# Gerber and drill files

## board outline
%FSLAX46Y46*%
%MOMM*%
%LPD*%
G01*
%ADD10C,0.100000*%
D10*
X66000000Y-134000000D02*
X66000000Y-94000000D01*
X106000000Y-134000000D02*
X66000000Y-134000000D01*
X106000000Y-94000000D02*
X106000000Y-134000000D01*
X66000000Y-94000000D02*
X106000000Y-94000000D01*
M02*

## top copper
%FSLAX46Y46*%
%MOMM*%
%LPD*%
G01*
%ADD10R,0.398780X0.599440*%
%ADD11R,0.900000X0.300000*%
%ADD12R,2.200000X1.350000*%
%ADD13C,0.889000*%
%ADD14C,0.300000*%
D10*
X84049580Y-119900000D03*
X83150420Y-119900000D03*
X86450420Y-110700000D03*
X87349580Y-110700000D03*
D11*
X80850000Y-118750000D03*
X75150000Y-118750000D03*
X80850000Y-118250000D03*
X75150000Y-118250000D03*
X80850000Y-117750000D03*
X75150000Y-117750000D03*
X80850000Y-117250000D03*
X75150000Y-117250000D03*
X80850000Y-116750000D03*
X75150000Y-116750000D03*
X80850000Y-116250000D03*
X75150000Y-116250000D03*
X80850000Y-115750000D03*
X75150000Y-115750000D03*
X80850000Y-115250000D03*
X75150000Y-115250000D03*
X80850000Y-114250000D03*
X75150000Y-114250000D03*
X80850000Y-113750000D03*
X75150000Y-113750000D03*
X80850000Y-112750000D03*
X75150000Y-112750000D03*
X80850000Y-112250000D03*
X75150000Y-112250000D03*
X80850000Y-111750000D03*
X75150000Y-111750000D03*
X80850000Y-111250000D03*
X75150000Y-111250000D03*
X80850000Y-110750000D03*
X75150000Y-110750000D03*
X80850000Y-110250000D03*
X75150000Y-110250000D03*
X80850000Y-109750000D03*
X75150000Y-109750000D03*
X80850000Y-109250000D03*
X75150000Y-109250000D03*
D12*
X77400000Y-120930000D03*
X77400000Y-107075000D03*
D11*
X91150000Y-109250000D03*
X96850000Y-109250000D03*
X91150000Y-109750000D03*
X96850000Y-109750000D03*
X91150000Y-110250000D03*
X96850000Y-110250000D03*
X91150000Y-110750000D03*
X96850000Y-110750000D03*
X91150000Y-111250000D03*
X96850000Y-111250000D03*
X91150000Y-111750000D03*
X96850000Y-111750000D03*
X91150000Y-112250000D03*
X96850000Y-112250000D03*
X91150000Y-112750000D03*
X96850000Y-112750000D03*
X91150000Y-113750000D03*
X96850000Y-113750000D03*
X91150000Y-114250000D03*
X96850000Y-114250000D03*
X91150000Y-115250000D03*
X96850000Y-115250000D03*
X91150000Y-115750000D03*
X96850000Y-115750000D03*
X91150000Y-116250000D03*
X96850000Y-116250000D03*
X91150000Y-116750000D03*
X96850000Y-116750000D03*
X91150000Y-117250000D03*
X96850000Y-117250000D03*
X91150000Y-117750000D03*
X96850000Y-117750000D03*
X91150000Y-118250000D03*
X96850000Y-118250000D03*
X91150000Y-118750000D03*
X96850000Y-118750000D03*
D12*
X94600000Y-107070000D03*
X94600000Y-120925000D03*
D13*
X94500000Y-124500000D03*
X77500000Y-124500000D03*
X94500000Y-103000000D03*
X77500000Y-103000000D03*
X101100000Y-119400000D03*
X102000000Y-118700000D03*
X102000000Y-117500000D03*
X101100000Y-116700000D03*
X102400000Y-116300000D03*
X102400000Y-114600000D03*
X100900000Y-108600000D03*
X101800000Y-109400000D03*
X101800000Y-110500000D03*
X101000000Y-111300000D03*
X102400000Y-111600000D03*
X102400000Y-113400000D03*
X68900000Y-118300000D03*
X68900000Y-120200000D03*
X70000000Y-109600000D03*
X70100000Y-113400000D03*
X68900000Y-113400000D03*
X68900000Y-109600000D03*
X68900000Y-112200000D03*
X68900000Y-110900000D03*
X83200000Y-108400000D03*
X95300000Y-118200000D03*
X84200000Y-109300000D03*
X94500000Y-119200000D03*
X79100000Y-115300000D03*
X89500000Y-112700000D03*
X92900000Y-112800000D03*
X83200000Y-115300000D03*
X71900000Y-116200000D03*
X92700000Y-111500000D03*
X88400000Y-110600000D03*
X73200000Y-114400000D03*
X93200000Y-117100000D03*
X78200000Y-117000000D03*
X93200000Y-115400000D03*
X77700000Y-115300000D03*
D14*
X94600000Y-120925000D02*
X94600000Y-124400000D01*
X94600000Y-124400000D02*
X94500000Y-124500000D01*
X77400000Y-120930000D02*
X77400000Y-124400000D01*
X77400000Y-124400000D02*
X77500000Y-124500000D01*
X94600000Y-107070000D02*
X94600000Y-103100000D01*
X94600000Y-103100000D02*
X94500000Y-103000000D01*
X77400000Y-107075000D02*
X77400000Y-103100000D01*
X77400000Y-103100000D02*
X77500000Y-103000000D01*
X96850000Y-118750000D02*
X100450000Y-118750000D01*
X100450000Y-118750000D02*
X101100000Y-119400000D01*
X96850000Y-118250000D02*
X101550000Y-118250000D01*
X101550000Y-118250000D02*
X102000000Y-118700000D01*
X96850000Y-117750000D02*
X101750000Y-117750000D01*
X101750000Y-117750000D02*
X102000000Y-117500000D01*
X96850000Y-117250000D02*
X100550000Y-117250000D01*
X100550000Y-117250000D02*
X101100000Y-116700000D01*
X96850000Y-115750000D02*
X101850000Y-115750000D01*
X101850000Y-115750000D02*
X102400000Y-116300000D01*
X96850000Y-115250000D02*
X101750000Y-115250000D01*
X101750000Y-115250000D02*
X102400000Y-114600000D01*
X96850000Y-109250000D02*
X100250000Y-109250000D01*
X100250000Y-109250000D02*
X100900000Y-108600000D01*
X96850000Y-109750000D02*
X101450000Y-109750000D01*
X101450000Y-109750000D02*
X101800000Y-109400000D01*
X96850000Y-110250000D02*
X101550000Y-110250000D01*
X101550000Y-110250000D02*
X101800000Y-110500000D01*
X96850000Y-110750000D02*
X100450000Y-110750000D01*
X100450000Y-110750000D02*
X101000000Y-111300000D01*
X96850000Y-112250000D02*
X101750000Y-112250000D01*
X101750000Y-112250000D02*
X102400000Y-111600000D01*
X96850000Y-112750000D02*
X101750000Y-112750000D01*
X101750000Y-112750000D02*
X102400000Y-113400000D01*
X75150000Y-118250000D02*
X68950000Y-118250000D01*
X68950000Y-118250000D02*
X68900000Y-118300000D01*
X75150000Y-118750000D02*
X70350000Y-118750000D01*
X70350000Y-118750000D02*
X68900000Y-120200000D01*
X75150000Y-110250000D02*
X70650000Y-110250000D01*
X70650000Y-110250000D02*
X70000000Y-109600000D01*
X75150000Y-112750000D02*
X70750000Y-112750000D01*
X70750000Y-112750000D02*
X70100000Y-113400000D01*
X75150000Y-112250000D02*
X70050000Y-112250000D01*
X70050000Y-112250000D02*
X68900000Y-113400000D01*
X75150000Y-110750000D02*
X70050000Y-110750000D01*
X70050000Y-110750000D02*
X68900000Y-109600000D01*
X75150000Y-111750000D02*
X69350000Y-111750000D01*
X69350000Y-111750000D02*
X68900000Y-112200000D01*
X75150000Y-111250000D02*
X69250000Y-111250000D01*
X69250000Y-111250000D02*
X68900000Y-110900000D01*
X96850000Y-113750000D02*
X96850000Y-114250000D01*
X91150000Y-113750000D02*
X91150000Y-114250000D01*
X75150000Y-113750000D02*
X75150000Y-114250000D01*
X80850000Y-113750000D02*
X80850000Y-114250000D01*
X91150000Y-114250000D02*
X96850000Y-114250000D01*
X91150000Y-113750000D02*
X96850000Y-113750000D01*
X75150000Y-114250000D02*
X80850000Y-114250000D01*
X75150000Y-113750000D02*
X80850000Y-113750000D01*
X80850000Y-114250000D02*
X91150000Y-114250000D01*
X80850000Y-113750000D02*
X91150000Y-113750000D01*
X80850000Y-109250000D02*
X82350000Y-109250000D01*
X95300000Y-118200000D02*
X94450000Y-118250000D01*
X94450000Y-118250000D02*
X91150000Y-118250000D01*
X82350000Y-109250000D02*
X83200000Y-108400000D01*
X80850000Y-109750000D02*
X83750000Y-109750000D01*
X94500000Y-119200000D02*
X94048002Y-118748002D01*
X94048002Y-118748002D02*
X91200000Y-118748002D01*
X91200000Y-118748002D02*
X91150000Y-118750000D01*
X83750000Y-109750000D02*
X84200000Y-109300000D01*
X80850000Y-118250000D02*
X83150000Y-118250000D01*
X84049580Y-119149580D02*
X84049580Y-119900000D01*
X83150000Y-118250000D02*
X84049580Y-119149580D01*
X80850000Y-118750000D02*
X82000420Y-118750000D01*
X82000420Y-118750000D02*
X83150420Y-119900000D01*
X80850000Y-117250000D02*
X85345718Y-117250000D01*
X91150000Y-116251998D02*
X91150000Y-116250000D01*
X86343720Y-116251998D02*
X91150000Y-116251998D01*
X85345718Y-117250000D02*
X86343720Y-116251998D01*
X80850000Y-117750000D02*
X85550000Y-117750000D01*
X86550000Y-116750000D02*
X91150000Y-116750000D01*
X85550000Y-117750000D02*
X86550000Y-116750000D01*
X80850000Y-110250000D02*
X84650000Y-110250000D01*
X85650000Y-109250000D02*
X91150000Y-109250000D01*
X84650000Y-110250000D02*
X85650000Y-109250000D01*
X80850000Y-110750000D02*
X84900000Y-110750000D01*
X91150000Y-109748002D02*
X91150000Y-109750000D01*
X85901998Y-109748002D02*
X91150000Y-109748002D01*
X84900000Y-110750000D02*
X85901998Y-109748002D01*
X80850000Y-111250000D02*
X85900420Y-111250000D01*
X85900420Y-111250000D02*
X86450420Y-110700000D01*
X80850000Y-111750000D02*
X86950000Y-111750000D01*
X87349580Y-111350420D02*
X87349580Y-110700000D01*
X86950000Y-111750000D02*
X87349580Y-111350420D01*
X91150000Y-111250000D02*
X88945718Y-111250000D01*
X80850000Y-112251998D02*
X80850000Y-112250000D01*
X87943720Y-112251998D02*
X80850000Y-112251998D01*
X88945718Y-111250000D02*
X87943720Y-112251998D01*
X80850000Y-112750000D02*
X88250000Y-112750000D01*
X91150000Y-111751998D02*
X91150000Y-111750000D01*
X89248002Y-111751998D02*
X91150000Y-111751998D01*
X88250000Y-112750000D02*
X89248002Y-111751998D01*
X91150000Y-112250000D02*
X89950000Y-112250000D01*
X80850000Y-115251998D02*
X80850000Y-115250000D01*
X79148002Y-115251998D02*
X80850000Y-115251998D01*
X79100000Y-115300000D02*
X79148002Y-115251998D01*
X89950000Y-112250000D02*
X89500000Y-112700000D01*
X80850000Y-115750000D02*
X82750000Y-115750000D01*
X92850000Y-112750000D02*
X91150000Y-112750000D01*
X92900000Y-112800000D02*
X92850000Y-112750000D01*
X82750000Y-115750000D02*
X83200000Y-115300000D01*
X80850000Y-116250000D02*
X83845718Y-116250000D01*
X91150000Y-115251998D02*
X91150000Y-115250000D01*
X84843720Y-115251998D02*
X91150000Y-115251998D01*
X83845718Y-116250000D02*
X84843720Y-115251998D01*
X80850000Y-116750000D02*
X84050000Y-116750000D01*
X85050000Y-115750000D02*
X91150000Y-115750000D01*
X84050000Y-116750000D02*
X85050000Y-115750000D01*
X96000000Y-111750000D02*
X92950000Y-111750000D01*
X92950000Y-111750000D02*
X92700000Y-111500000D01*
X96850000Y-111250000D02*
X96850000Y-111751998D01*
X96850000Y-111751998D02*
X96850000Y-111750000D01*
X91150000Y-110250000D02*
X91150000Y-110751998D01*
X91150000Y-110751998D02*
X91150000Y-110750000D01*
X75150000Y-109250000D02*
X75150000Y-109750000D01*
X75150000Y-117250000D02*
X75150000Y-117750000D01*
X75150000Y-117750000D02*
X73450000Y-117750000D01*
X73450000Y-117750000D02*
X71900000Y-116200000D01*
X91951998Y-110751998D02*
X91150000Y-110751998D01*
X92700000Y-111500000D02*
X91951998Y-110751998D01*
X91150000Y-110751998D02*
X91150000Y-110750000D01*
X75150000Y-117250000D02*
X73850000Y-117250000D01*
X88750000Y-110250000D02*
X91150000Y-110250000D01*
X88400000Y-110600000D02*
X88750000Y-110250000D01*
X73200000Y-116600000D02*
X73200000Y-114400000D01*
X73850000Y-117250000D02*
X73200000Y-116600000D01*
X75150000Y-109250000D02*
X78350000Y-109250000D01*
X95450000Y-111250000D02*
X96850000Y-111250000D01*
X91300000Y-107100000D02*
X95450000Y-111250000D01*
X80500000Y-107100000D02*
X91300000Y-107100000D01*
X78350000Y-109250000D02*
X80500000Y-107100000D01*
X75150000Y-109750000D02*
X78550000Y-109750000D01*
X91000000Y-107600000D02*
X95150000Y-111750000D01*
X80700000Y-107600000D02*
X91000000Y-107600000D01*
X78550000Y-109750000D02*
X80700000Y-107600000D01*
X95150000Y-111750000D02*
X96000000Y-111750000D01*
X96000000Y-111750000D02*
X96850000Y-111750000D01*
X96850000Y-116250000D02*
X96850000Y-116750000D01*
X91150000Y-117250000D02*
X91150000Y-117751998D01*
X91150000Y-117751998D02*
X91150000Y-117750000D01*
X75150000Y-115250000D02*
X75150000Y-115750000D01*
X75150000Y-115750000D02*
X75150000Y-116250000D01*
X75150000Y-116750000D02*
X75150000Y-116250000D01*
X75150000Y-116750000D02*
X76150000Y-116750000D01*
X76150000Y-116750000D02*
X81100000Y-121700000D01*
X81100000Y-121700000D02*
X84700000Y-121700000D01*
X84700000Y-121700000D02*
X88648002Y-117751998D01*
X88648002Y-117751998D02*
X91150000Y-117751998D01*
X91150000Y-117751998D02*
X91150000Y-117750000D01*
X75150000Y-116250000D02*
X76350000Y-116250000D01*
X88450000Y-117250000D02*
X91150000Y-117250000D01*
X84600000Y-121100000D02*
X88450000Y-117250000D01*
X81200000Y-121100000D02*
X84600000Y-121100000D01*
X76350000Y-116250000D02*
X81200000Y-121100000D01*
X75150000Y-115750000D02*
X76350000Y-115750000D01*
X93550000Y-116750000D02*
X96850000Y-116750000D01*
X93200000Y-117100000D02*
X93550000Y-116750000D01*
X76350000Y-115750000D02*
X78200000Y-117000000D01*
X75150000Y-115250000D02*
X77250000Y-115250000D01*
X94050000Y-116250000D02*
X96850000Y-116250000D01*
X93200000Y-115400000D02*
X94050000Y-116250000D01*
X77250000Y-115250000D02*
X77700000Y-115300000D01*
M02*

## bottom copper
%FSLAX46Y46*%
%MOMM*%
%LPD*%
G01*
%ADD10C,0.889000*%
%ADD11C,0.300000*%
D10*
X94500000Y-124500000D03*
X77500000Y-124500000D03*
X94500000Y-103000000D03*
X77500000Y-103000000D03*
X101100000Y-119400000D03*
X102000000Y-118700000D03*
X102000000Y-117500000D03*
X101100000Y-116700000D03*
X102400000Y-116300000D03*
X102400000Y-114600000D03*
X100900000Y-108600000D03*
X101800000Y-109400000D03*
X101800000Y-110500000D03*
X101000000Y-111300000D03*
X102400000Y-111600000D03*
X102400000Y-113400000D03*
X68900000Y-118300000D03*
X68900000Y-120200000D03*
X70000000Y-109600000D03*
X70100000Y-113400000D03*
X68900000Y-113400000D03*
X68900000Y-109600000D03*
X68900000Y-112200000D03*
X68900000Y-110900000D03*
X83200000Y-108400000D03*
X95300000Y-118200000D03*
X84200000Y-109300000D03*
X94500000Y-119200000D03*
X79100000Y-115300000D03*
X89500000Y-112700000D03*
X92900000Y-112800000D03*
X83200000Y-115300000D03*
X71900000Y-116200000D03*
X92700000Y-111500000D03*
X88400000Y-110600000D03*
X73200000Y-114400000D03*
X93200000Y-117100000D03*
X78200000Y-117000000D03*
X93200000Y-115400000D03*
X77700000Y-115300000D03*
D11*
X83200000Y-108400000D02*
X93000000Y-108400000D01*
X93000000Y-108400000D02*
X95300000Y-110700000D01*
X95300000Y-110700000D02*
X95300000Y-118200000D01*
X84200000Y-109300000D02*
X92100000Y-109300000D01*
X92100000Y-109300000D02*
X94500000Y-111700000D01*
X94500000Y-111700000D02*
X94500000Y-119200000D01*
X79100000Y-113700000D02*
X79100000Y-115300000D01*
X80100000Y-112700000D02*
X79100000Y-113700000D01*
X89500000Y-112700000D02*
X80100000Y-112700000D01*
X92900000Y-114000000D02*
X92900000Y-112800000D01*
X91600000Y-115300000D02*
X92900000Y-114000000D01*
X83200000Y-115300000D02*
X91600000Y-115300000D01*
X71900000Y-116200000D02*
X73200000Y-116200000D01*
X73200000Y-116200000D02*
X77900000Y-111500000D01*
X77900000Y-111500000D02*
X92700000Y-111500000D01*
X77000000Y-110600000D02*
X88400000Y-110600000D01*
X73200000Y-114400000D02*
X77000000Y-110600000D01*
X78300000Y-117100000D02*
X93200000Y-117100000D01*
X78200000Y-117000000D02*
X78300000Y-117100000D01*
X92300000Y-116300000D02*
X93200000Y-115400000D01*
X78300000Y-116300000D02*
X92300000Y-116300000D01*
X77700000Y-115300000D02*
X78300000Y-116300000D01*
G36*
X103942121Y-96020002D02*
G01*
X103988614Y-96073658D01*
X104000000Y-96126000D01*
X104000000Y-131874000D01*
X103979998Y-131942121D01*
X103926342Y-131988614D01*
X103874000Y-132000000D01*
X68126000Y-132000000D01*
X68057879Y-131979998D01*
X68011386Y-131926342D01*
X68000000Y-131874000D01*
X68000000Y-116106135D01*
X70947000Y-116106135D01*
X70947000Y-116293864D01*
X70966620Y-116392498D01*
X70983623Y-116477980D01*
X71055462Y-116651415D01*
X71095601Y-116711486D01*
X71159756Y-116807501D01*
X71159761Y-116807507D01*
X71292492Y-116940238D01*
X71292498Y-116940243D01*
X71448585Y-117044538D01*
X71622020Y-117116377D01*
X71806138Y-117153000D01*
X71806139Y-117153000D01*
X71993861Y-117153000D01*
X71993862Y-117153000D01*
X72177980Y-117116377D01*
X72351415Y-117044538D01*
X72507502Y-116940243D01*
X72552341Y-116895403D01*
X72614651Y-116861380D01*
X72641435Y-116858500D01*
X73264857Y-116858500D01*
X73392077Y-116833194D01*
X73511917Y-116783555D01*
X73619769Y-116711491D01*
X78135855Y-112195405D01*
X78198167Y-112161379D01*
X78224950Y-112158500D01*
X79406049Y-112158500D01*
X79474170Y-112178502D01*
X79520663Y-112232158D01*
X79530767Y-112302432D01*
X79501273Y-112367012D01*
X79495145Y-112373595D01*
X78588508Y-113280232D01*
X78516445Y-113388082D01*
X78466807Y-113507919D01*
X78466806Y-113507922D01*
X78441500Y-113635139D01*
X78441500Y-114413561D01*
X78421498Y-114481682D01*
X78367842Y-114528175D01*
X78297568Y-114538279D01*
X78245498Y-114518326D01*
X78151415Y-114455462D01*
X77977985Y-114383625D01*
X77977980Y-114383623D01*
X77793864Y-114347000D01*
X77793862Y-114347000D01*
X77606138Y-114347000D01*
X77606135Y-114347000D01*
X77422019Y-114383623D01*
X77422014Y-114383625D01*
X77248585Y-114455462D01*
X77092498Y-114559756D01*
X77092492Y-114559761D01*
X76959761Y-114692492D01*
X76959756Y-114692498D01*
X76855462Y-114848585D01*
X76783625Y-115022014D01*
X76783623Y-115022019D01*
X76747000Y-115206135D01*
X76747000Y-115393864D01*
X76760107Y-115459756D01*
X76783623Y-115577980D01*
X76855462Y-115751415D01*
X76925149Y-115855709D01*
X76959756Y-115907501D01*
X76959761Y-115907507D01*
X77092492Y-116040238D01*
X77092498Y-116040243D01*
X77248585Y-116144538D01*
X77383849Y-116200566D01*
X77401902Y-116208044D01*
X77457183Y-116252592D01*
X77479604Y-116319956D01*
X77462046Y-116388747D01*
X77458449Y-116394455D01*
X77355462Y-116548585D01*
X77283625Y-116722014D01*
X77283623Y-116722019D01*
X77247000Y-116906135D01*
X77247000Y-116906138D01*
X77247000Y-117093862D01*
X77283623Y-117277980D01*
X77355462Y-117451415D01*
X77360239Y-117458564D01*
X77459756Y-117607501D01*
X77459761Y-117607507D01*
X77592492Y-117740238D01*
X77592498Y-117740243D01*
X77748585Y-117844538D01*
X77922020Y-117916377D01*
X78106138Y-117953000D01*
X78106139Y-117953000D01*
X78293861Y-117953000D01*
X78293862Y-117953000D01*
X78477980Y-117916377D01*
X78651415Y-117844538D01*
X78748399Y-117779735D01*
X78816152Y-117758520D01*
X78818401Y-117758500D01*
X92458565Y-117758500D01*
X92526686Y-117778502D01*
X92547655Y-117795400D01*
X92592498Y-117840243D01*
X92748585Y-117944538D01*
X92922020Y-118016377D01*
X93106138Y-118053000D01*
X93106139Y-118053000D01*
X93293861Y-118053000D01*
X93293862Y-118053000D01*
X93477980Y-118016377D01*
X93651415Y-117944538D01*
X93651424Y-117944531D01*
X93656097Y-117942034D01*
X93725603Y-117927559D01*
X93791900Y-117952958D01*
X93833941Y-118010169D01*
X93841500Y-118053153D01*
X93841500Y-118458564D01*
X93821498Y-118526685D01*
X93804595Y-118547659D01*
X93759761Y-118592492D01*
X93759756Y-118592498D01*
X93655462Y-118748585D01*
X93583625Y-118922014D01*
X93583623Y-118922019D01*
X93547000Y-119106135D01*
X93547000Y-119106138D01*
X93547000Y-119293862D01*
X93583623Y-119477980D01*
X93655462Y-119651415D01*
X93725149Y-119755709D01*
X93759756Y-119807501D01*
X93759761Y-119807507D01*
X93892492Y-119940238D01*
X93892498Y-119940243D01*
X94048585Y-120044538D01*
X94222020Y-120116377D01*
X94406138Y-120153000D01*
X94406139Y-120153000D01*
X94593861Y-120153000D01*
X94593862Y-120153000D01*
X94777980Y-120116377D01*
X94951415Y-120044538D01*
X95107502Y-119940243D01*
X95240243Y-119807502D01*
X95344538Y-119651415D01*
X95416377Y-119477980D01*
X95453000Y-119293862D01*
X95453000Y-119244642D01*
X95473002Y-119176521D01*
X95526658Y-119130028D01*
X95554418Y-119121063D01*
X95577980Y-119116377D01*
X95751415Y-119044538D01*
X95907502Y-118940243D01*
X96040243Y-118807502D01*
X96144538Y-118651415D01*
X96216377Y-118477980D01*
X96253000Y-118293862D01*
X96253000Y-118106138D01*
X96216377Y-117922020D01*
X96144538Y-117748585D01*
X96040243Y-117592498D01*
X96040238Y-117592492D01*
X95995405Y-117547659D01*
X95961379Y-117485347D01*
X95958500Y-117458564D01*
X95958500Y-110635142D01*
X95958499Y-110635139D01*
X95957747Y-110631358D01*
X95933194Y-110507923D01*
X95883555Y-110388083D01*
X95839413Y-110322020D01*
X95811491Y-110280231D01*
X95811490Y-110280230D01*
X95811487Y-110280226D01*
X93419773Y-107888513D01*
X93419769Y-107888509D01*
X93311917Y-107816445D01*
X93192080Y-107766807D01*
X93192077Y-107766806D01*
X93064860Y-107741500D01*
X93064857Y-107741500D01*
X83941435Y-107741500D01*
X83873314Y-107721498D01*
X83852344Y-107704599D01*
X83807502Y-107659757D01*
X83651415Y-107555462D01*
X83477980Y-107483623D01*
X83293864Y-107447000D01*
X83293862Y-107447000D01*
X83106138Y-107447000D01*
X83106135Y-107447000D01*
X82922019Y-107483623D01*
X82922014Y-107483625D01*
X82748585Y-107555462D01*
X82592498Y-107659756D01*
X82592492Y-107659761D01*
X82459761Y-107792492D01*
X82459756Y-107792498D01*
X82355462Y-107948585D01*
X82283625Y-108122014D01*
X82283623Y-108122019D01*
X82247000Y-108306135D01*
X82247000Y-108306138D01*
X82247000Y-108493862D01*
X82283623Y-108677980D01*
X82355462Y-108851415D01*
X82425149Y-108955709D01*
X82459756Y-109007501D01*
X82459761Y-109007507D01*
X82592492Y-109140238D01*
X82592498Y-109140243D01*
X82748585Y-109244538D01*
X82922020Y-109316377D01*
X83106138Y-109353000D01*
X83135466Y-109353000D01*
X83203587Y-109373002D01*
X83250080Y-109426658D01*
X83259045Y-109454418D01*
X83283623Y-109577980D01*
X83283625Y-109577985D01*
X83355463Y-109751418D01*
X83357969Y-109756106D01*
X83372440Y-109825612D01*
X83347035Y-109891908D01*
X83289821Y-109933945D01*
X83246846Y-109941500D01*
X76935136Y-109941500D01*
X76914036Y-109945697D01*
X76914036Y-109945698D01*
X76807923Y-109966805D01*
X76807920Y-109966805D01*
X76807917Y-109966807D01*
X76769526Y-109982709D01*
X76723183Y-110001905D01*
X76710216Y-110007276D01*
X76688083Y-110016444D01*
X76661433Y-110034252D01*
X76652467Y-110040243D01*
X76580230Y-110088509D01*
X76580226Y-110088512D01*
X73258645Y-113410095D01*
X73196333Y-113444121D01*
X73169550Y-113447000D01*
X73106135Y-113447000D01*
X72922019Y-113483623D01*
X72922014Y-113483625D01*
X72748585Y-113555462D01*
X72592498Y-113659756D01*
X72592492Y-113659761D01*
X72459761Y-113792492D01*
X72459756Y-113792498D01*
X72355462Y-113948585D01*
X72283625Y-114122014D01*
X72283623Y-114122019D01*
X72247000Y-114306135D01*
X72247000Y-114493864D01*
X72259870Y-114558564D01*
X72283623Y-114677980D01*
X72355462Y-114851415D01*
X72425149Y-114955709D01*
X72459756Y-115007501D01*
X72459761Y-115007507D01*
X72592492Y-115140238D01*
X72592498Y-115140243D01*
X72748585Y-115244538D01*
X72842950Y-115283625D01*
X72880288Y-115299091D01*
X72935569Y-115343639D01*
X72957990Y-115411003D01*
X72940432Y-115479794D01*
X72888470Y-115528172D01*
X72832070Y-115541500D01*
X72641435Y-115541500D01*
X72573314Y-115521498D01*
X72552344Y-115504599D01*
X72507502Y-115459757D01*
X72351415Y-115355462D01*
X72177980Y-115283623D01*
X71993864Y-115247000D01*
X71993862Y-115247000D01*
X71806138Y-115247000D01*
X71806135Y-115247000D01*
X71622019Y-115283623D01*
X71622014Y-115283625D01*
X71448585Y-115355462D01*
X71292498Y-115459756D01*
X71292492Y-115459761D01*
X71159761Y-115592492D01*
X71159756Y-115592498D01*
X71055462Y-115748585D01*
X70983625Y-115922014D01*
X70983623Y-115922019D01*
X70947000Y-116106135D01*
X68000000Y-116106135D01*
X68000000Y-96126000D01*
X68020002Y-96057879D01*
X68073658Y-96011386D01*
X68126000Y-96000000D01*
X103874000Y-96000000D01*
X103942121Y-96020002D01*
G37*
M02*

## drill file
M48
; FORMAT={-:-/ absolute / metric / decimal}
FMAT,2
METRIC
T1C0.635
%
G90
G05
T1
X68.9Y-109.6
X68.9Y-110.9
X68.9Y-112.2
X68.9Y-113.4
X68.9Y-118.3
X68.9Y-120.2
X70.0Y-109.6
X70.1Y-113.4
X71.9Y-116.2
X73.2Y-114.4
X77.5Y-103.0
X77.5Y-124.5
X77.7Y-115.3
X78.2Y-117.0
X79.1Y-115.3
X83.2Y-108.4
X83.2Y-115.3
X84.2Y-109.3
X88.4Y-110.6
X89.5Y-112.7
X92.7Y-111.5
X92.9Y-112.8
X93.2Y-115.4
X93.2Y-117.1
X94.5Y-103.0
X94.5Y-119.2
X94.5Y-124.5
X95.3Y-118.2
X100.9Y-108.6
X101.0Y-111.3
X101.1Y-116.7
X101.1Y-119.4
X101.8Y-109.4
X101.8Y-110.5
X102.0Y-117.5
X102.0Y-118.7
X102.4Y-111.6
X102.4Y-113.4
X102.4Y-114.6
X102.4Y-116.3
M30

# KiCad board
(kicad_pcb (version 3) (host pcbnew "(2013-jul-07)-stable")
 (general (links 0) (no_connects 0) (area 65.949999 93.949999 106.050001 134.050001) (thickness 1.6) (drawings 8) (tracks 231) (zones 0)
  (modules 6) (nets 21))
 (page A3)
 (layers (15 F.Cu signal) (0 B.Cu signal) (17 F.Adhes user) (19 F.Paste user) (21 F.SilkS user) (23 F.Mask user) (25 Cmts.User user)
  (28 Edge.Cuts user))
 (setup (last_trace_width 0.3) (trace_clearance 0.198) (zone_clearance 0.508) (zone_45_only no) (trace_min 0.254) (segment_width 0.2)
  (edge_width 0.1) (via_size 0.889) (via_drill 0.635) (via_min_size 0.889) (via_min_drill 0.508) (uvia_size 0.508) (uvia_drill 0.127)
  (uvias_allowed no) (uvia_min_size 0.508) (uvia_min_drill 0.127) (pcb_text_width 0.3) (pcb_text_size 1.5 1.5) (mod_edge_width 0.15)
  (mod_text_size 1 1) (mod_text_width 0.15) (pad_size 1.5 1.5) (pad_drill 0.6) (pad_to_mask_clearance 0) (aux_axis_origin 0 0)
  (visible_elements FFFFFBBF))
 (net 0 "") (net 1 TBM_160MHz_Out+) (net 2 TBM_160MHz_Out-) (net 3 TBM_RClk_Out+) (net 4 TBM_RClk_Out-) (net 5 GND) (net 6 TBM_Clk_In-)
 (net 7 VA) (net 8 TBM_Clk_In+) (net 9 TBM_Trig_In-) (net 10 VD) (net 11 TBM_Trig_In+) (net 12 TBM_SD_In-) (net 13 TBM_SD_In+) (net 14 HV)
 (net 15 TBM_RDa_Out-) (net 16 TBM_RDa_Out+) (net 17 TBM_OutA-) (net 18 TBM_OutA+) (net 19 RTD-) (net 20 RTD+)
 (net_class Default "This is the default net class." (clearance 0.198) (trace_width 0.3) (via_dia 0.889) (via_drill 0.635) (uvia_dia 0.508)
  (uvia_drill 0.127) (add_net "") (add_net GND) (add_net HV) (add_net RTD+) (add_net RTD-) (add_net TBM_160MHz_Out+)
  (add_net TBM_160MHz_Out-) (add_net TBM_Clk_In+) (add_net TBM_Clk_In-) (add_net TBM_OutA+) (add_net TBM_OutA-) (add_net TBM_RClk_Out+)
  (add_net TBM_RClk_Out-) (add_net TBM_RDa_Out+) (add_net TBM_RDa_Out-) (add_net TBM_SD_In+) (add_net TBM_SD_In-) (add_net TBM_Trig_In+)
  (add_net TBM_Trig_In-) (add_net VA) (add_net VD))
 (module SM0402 (layer F.Cu) (at 83.6 119.9 180)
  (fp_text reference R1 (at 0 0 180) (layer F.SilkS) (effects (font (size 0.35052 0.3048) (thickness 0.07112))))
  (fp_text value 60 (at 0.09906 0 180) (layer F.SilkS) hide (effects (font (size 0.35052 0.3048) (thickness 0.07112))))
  (pad 1 smd rect (at -0.44958 0 180) (size 0.39878 0.59944) (layers F.Cu F.Paste F.Mask) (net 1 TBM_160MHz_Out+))
  (pad 2 smd rect (at 0.44958 0 180) (size 0.39878 0.59944) (layers F.Cu F.Paste F.Mask) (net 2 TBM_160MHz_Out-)))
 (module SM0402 (layer F.Cu) (at 86.9 110.7)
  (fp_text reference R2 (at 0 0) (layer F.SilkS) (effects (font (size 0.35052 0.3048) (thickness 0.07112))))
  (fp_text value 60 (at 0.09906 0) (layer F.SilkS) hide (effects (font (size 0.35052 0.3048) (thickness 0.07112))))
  (pad 1 smd rect (at -0.44958 0) (size 0.39878 0.59944) (layers F.Cu F.Paste F.Mask) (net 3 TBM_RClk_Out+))
  (pad 2 smd rect (at 0.44958 0) (size 0.39878 0.59944) (layers F.Cu F.Paste F.Mask) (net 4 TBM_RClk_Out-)))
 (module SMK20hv (layer F.Cu) (at 78 114 90)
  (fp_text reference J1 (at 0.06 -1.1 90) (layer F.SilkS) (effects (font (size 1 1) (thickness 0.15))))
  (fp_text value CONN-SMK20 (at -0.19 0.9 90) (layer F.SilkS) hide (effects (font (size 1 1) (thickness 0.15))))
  (pad 1 smd rect (at -4.75 2.85 90) (size 0.3 0.9) (layers F.Cu F.Paste F.Mask) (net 2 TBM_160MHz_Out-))
  (pad 2 smd rect (at -4.75 -2.85 90) (size 0.3 0.9) (layers F.Cu F.Paste F.Mask) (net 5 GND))
  (pad 3 smd rect (at -4.25 2.85 90) (size 0.3 0.9) (layers F.Cu F.Paste F.Mask) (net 1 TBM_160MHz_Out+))
  (pad 4 smd rect (at -4.25 -2.85 90) (size 0.3 0.9) (layers F.Cu F.Paste F.Mask) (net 5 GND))
  (pad 5 smd rect (at -3.75 2.85 90) (size 0.3 0.9) (layers F.Cu F.Paste F.Mask) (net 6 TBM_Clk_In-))
  (pad 6 smd rect (at -3.75 -2.85 90) (size 0.3 0.9) (layers F.Cu F.Paste F.Mask) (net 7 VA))
  (pad 7 smd rect (at -3.25 2.85 90) (size 0.3 0.9) (layers F.Cu F.Paste F.Mask) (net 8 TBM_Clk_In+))
  (pad 8 smd rect (at -3.25 -2.85 90) (size 0.3 0.9) (layers F.Cu F.Paste F.Mask) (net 7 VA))
  (pad 9 smd rect (at -2.75 2.85 90) (size 0.3 0.9) (layers F.Cu F.Paste F.Mask) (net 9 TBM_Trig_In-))
  (pad 10 smd rect (at -2.75 -2.85 90) (size 0.3 0.9) (layers F.Cu F.Paste F.Mask) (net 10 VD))
  (pad 11 smd rect (at -2.25 2.85 90) (size 0.3 0.9) (layers F.Cu F.Paste F.Mask) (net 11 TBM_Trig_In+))
  (pad 12 smd rect (at -2.25 -2.85 90) (size 0.3 0.9) (layers F.Cu F.Paste F.Mask) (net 10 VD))
  (pad 13 smd rect (at -1.75 2.85 90) (size 0.3 0.9) (layers F.Cu F.Paste F.Mask) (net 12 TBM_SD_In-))
  (pad 14 smd rect (at -1.75 -2.85 90) (size 0.3 0.9) (layers F.Cu F.Paste F.Mask) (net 10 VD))
  (pad 15 smd rect (at -1.25 2.85 90) (size 0.3 0.9) (layers F.Cu F.Paste F.Mask) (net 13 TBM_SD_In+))
  (pad 16 smd rect (at -1.25 -2.85 90) (size 0.3 0.9) (layers F.Cu F.Paste F.Mask) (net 10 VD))
  (pad 19 smd rect (at -0.25 2.85 90) (size 0.3 0.9) (layers F.Cu F.Paste F.Mask) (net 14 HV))
  (pad 20 smd rect (at -0.25 -2.85 90) (size 0.3 0.9) (layers F.Cu F.Paste F.Mask) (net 14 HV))
  (pad 21 smd rect (at 0.25 2.85 90) (size 0.3 0.9) (layers F.Cu F.Paste F.Mask) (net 14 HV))
  (pad 22 smd rect (at 0.25 -2.85 90) (size 0.3 0.9) (layers F.Cu F.Paste F.Mask) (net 14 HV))
  (pad 25 smd rect (at 1.25 2.85 90) (size 0.3 0.9) (layers F.Cu F.Paste F.Mask) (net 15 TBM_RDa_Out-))
  (pad 26 smd rect (at 1.25 -2.85 90) (size 0.3 0.9) (layers F.Cu F.Paste F.Mask) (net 5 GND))
  (pad 27 smd rect (at 1.75 2.85 90) (size 0.3 0.9) (layers F.Cu F.Paste F.Mask) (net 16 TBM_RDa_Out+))
  (pad 28 smd rect (at 1.75 -2.85 90) (size 0.3 0.9) (layers F.Cu F.Paste F.Mask) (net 5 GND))
  (pad 29 smd rect (at 2.25 2.85 90) (size 0.3 0.9) (layers F.Cu F.Paste F.Mask) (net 4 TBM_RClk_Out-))
  (pad 30 smd rect (at 2.25 -2.85 90) (size 0.3 0.9) (layers F.Cu F.Paste F.Mask) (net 5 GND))
  (pad 31 smd rect (at 2.75 2.85 90) (size 0.3 0.9) (layers F.Cu F.Paste F.Mask) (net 3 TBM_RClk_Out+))
  (pad 32 smd rect (at 2.75 -2.85 90) (size 0.3 0.9) (layers F.Cu F.Paste F.Mask) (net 5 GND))
  (pad 33 smd rect (at 3.25 2.85 90) (size 0.3 0.9) (layers F.Cu F.Paste F.Mask) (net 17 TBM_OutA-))
  (pad 34 smd rect (at 3.25 -2.85 90) (size 0.3 0.9) (layers F.Cu F.Paste F.Mask) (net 5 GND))
  (pad 35 smd rect (at 3.75 2.85 90) (size 0.3 0.9) (layers F.Cu F.Paste F.Mask) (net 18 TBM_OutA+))
  (pad 36 smd rect (at 3.75 -2.85 90) (size 0.3 0.9) (layers F.Cu F.Paste F.Mask) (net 5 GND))
  (pad 37 smd rect (at 4.25 2.85 90) (size 0.3 0.9) (layers F.Cu F.Paste F.Mask) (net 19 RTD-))
  (pad 38 smd rect (at 4.25 -2.85 90) (size 0.3 0.9) (layers F.Cu F.Paste F.Mask) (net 7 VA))
  (pad 39 smd rect (at 4.75 2.85 90) (size 0.3 0.9) (layers F.Cu F.Paste F.Mask) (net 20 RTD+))
  (pad 40 smd rect (at 4.75 -2.85 90) (size 0.3 0.9) (layers F.Cu F.Paste F.Mask) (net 7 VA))
  (pad 41 smd rect (at -6.93 -0.6 90) (size 1.35 2.2) (layers F.Cu F.Paste F.Mask) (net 5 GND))
  (pad 42 smd rect (at 6.925 -0.6 90) (size 1.35 2.2) (layers F.Cu F.Paste F.Mask) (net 5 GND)))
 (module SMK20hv (layer F.Cu) (at 94 114 270)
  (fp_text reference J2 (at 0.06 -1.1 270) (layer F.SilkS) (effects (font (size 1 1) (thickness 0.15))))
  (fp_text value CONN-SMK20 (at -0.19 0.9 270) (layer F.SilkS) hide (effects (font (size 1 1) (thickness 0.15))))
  (pad 1 smd rect (at -4.75 2.85 270) (size 0.3 0.9) (layers F.Cu F.Paste F.Mask) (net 18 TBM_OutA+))
  (pad 2 smd rect (at -4.75 -2.85 270) (size 0.3 0.9) (layers F.Cu F.Paste F.Mask) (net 5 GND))
  (pad 3 smd rect (at -4.25 2.85 270) (size 0.3 0.9) (layers F.Cu F.Paste F.Mask) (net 17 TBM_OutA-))
  (pad 4 smd rect (at -4.25 -2.85 270) (size 0.3 0.9) (layers F.Cu F.Paste F.Mask) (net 5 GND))
  (pad 5 smd rect (at -3.75 2.85 270) (size 0.3 0.9) (layers F.Cu F.Paste F.Mask) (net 7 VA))
  (pad 6 smd rect (at -3.75 -2.85 270) (size 0.3 0.9) (layers F.Cu F.Paste F.Mask) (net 5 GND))
  (pad 7 smd rect (at -3.25 2.85 270) (size 0.3 0.9) (layers F.Cu F.Paste F.Mask) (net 7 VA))
  (pad 8 smd rect (at -3.25 -2.85 270) (size 0.3 0.9) (layers F.Cu F.Paste F.Mask) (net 5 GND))
  (pad 9 smd rect (at -2.75 2.85 270) (size 0.3 0.9) (layers F.Cu F.Paste F.Mask) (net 16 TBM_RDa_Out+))
  (pad 10 smd rect (at -2.75 -2.85 270) (size 0.3 0.9) (layers F.Cu F.Paste F.Mask) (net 7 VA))
  (pad 11 smd rect (at -2.25 2.85 270) (size 0.3 0.9) (layers F.Cu F.Paste F.Mask) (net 15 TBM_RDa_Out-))
  (pad 12 smd rect (at -2.25 -2.85 270) (size 0.3 0.9) (layers F.Cu F.Paste F.Mask) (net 7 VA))
  (pad 13 smd rect (at -1.75 2.85 270) (size 0.3 0.9) (layers F.Cu F.Paste F.Mask) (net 13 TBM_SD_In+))
  (pad 14 smd rect (at -1.75 -2.85 270) (size 0.3 0.9) (layers F.Cu F.Paste F.Mask) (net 5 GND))
  (pad 15 smd rect (at -1.25 2.85 270) (size 0.3 0.9) (layers F.Cu F.Paste F.Mask) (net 12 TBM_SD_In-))
  (pad 16 smd rect (at -1.25 -2.85 270) (size 0.3 0.9) (layers F.Cu F.Paste F.Mask) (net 5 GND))
  (pad 19 smd rect (at -0.25 2.85 270) (size 0.3 0.9) (layers F.Cu F.Paste F.Mask) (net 14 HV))
  (pad 20 smd rect (at -0.25 -2.85 270) (size 0.3 0.9) (layers F.Cu F.Paste F.Mask) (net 14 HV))
  (pad 21 smd rect (at 0.25 2.85 270) (size 0.3 0.9) (layers F.Cu F.Paste F.Mask) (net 14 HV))
  (pad 22 smd rect (at 0.25 -2.85 270) (size 0.3 0.9) (layers F.Cu F.Paste F.Mask) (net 14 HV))
  (pad 25 smd rect (at 1.25 2.85 270) (size 0.3 0.9) (layers F.Cu F.Paste F.Mask) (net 11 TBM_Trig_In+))
  (pad 26 smd rect (at 1.25 -2.85 270) (size 0.3 0.9) (layers F.Cu F.Paste F.Mask) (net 5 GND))
  (pad 27 smd rect (at 1.75 2.85 270) (size 0.3 0.9) (layers F.Cu F.Paste F.Mask) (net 9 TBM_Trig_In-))
  (pad 28 smd rect (at 1.75 -2.85 270) (size 0.3 0.9) (layers F.Cu F.Paste F.Mask) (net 5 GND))
  (pad 29 smd rect (at 2.25 2.85 270) (size 0.3 0.9) (layers F.Cu F.Paste F.Mask) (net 8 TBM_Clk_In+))
  (pad 30 smd rect (at 2.25 -2.85 270) (size 0.3 0.9) (layers F.Cu F.Paste F.Mask) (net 10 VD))
  (pad 31 smd rect (at 2.75 2.85 270) (size 0.3 0.9) (layers F.Cu F.Paste F.Mask) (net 6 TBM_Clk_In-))
  (pad 32 smd rect (at 2.75 -2.85 270) (size 0.3 0.9) (layers F.Cu F.Paste F.Mask) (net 10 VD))
  (pad 33 smd rect (at 3.25 2.85 270) (size 0.3 0.9) (layers F.Cu F.Paste F.Mask) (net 10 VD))
  (pad 34 smd rect (at 3.25 -2.85 270) (size 0.3 0.9) (layers F.Cu F.Paste F.Mask) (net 5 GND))
  (pad 35 smd rect (at 3.75 2.85 270) (size 0.3 0.9) (layers F.Cu F.Paste F.Mask) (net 10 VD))
  (pad 36 smd rect (at 3.75 -2.85 270) (size 0.3 0.9) (layers F.Cu F.Paste F.Mask) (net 5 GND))
  (pad 37 smd rect (at 4.25 2.85 270) (size 0.3 0.9) (layers F.Cu F.Paste F.Mask) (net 20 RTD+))
  (pad 38 smd rect (at 4.25 -2.85 270) (size 0.3 0.9) (layers F.Cu F.Paste F.Mask) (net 5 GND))
  (pad 39 smd rect (at 4.75 2.85 270) (size 0.3 0.9) (layers F.Cu F.Paste F.Mask) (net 19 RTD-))
  (pad 40 smd rect (at 4.75 -2.85 270) (size 0.3 0.9) (layers F.Cu F.Paste F.Mask) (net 5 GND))
  (pad 41 smd rect (at -6.93 -0.6 270) (size 1.35 2.2) (layers F.Cu F.Paste F.Mask) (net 5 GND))
  (pad 42 smd rect (at 6.925 -0.6 270) (size 1.35 2.2) (layers F.Cu F.Paste F.Mask) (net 5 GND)))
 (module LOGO (layer F.Cu) (at 101 100)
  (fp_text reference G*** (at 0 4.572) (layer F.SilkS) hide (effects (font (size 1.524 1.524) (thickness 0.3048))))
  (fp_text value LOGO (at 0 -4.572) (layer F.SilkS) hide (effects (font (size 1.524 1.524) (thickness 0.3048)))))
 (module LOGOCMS (layer F.Cu) (at 71.5 100)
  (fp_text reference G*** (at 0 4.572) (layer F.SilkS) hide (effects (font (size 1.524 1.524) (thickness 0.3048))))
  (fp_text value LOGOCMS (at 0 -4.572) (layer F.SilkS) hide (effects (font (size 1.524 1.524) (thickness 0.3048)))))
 (gr_line (start 66 134) (end 66 94) (angle 90) (layer Edge.Cuts) (width 0.1))
 (gr_line (start 106 134) (end 66 134) (angle 90) (layer Edge.Cuts) (width 0.1))
 (gr_line (start 106 94) (end 106 134) (angle 90) (layer Edge.Cuts) (width 0.1))
 (gr_line (start 66 94) (end 106 94) (angle 90) (layer Edge.Cuts) (width 0.1))
 (segment (start 94.6 120.925) (end 94.6 124.4) (width 0.3) (layer F.Cu) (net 5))
 (via (at 94.5 124.5) (size 0.889) (layers F.Cu B.Cu) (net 5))
 (segment (start 94.6 124.4) (end 94.5 124.5) (width 0.3) (layer F.Cu) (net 5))
 (segment (start 77.4 120.93) (end 77.4 124.4) (width 0.3) (layer F.Cu) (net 5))
 (via (at 77.5 124.5) (size 0.889) (layers F.Cu B.Cu) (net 5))
 (segment (start 77.4 124.4) (end 77.5 124.5) (width 0.3) (layer F.Cu) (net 5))
 (segment (start 94.6 107.07) (end 94.6 103.1) (width 0.3) (layer F.Cu) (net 5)) (via (at 94.5 103) (size 0.889) (layers F.Cu B.Cu) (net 5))
 (segment (start 94.6 103.1) (end 94.5 103) (width 0.3) (layer F.Cu) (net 5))
 (segment (start 77.4 107.075) (end 77.4 103.1) (width 0.3) (layer F.Cu) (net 5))
 (via (at 77.5 103) (size 0.889) (layers F.Cu B.Cu) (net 5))
 (segment (start 77.4 103.1) (end 77.5 103) (width 0.3) (layer F.Cu) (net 5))
 (segment (start 96.85 118.75) (end 100.45 118.75) (width 0.3) (layer F.Cu) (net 5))
 (via (at 101.1 119.4) (size 0.889) (layers F.Cu B.Cu) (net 5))
 (segment (start 100.45 118.75) (end 101.1 119.4) (width 0.3) (layer F.Cu) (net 5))
 (segment (start 96.85 118.25) (end 101.55 118.25) (width 0.3) (layer F.Cu) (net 5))
 (via (at 102 118.7) (size 0.889) (layers F.Cu B.Cu) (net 5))
 (segment (start 101.55 118.25) (end 102 118.7) (width 0.3) (layer F.Cu) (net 5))
 (segment (start 96.85 117.75) (end 101.75 117.75) (width 0.3) (layer F.Cu) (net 5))
 (via (at 102 117.5) (size 0.889) (layers F.Cu B.Cu) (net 5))
 (segment (start 101.75 117.75) (end 102 117.5) (width 0.3) (layer F.Cu) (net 5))
 (segment (start 96.85 117.25) (end 100.55 117.25) (width 0.3) (layer F.Cu) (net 5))
 (via (at 101.1 116.7) (size 0.889) (layers F.Cu B.Cu) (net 5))
 (segment (start 100.55 117.25) (end 101.1 116.7) (width 0.3) (layer F.Cu) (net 5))
 (segment (start 96.85 115.75) (end 101.85 115.75) (width 0.3) (layer F.Cu) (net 5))
 (via (at 102.4 116.3) (size 0.889) (layers F.Cu B.Cu) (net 5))
 (segment (start 101.85 115.75) (end 102.4 116.3) (width 0.3) (layer F.Cu) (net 5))
 (segment (start 96.85 115.25) (end 101.75 115.25) (width 0.3) (layer F.Cu) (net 5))
 (via (at 102.4 114.6) (size 0.889) (layers F.Cu B.Cu) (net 5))
 (segment (start 101.75 115.25) (end 102.4 114.6) (width 0.3) (layer F.Cu) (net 5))
 (segment (start 96.85 109.25) (end 100.25 109.25) (width 0.3) (layer F.Cu) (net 5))
 (via (at 100.9 108.6) (size 0.889) (layers F.Cu B.Cu) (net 5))
 (segment (start 100.25 109.25) (end 100.9 108.6) (width 0.3) (layer F.Cu) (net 5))
 (segment (start 96.85 109.75) (end 101.45 109.75) (width 0.3) (layer F.Cu) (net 5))
 (via (at 101.8 109.4) (size 0.889) (layers F.Cu B.Cu) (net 5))
 (segment (start 101.45 109.75) (end 101.8 109.4) (width 0.3) (layer F.Cu) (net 5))
 (segment (start 96.85 110.25) (end 101.55 110.25) (width 0.3) (layer F.Cu) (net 5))
 (via (at 101.8 110.5) (size 0.889) (layers F.Cu B.Cu) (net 5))
 (segment (start 101.55 110.25) (end 101.8 110.5) (width 0.3) (layer F.Cu) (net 5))
 (segment (start 96.85 110.75) (end 100.45 110.75) (width 0.3) (layer F.Cu) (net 5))
 (via (at 101 111.3) (size 0.889) (layers F.Cu B.Cu) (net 5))
 (segment (start 100.45 110.75) (end 101 111.3) (width 0.3) (layer F.Cu) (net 5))
 (segment (start 96.85 112.25) (end 101.75 112.25) (width 0.3) (layer F.Cu) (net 5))
 (via (at 102.4 111.6) (size 0.889) (layers F.Cu B.Cu) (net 5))
 (segment (start 101.75 112.25) (end 102.4 111.6) (width 0.3) (layer F.Cu) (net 5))
 (segment (start 96.85 112.75) (end 101.75 112.75) (width 0.3) (layer F.Cu) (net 5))
 (via (at 102.4 113.4) (size 0.889) (layers F.Cu B.Cu) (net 5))
 (segment (start 101.75 112.75) (end 102.4 113.4) (width 0.3) (layer F.Cu) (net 5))
 (segment (start 75.15 118.25) (end 68.95 118.25) (width 0.3) (layer F.Cu) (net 5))
 (via (at 68.9 118.3) (size 0.889) (layers F.Cu B.Cu) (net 5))
 (segment (start 68.95 118.25) (end 68.9 118.3) (width 0.3) (layer F.Cu) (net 5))
 (segment (start 75.15 118.75) (end 70.35 118.75) (width 0.3) (layer F.Cu) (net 5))
 (via (at 68.9 120.2) (size 0.889) (layers F.Cu B.Cu) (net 5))
 (segment (start 70.35 118.75) (end 68.9 120.2) (width 0.3) (layer F.Cu) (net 5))
 (segment (start 75.15 110.25) (end 70.65 110.25) (width 0.3) (layer F.Cu) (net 5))
 (via (at 70 109.6) (size 0.889) (layers F.Cu B.Cu) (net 5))
 (segment (start 70.65 110.25) (end 70 109.6) (width 0.3) (layer F.Cu) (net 5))
 (segment (start 75.15 112.75) (end 70.75 112.75) (width 0.3) (layer F.Cu) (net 5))
 (via (at 70.1 113.4) (size 0.889) (layers F.Cu B.Cu) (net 5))
 (segment (start 70.75 112.75) (end 70.1 113.4) (width 0.3) (layer F.Cu) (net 5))
 (segment (start 75.15 112.25) (end 70.05 112.25) (width 0.3) (layer F.Cu) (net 5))
 (via (at 68.9 113.4) (size 0.889) (layers F.Cu B.Cu) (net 5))
 (segment (start 70.05 112.25) (end 68.9 113.4) (width 0.3) (layer F.Cu) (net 5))
 (segment (start 75.15 110.75) (end 70.05 110.75) (width 0.3) (layer F.Cu) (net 5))
 (via (at 68.9 109.6) (size 0.889) (layers F.Cu B.Cu) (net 5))
 (segment (start 70.05 110.75) (end 68.9 109.6) (width 0.3) (layer F.Cu) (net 5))
 (segment (start 75.15 111.75) (end 69.35 111.75) (width 0.3) (layer F.Cu) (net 5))
 (via (at 68.9 112.2) (size 0.889) (layers F.Cu B.Cu) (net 5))
 (segment (start 69.35 111.75) (end 68.9 112.2) (width 0.3) (layer F.Cu) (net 5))
 (segment (start 75.15 111.25) (end 69.25 111.25) (width 0.3) (layer F.Cu) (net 5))
 (via (at 68.9 110.9) (size 0.889) (layers F.Cu B.Cu) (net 5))
 (segment (start 69.25 111.25) (end 68.9 110.9) (width 0.3) (layer F.Cu) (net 5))
 (segment (start 96.85 113.75) (end 96.85 114.25) (width 0.3) (layer F.Cu) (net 14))
 (segment (start 91.15 113.75) (end 91.15 114.25) (width 0.3) (layer F.Cu) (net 14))
 (segment (start 75.15 113.75) (end 75.15 114.25) (width 0.3) (layer F.Cu) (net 14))
 (segment (start 80.85 113.75) (end 80.85 114.25) (width 0.3) (layer F.Cu) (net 14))
 (segment (start 91.15 114.25) (end 96.85 114.25) (width 0.3) (layer F.Cu) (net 14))
 (segment (start 91.15 113.75) (end 96.85 113.75) (width 0.3) (layer F.Cu) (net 14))
 (segment (start 75.15 114.25) (end 80.85 114.25) (width 0.3) (layer F.Cu) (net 14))
 (segment (start 75.15 113.75) (end 80.85 113.75) (width 0.3) (layer F.Cu) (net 14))
 (segment (start 80.85 114.25) (end 91.15 114.25) (width 0.3) (layer F.Cu) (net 14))
 (segment (start 80.85 113.75) (end 91.15 113.75) (width 0.3) (layer F.Cu) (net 14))
 (segment (start 80.85 109.25) (end 82.35 109.25) (width 0.3) (layer F.Cu) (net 20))
 (via (at 83.2 108.4) (size 0.889) (layers F.Cu B.Cu) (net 20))
 (segment (start 83.2 108.4) (end 93 108.4) (width 0.3) (layer B.Cu) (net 20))
 (segment (start 93 108.4) (end 95.3 110.7) (width 0.3) (layer B.Cu) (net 20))
 (segment (start 95.3 110.7) (end 95.3 118.2) (width 0.3) (layer B.Cu) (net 20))
 (via (at 95.3 118.2) (size 0.889) (layers F.Cu B.Cu) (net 20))
 (segment (start 95.3 118.2) (end 94.45 118.25) (width 0.3) (layer F.Cu) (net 20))
 (segment (start 94.45 118.25) (end 91.15 118.25) (width 0.3) (layer F.Cu) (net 20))
 (segment (start 82.35 109.25) (end 83.2 108.4) (width 0.3) (layer F.Cu) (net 20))
 (segment (start 80.85 109.75) (end 83.75 109.75) (width 0.3) (layer F.Cu) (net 19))
 (via (at 84.2 109.3) (size 0.889) (layers F.Cu B.Cu) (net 19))
 (segment (start 84.2 109.3) (end 92.1 109.3) (width 0.3) (layer B.Cu) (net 19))
 (segment (start 92.1 109.3) (end 94.5 111.7) (width 0.3) (layer B.Cu) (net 19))
 (segment (start 94.5 111.7) (end 94.5 119.2) (width 0.3) (layer B.Cu) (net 19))
 (via (at 94.5 119.2) (size 0.889) (layers F.Cu B.Cu) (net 19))
 (segment (start 94.5 119.2) (end 94.048002 118.748002) (width 0.3) (layer F.Cu) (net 19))
 (segment (start 94.048002 118.748002) (end 91.2 118.748002) (width 0.3) (layer F.Cu) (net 19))
 (segment (start 91.2 118.748002) (end 91.15 118.75) (width 0.3) (layer F.Cu) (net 19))
 (segment (start 83.75 109.75) (end 84.2 109.3) (width 0.3) (layer F.Cu) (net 19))
 (segment (start 80.85 118.25) (end 83.15 118.25) (width 0.3) (layer F.Cu) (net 1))
 (segment (start 84.04958 119.14958) (end 84.04958 119.9) (width 0.3) (layer F.Cu) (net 1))
 (segment (start 83.15 118.25) (end 84.04958 119.14958) (width 0.3) (layer F.Cu) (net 1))
 (segment (start 80.85 118.75) (end 82.00042 118.75) (width 0.3) (layer F.Cu) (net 2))
 (segment (start 82.00042 118.75) (end 83.15042 119.9) (width 0.3) (layer F.Cu) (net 2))
 (segment (start 80.85 117.25) (end 85.345718 117.25) (width 0.3) (layer F.Cu) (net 8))
 (segment (start 91.15 116.251998) (end 91.15 116.25) (width 0.3) (layer F.Cu) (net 8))
 (segment (start 86.34372 116.251998) (end 91.15 116.251998) (width 0.3) (layer F.Cu) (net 8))
 (segment (start 85.345718 117.25) (end 86.34372 116.251998) (width 0.3) (layer F.Cu) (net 8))
 (segment (start 80.85 117.75) (end 85.55 117.75) (width 0.3) (layer F.Cu) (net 6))
 (segment (start 86.55 116.75) (end 91.15 116.75) (width 0.3) (layer F.Cu) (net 6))
 (segment (start 85.55 117.75) (end 86.55 116.75) (width 0.3) (layer F.Cu) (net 6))
 (segment (start 80.85 110.25) (end 84.65 110.25) (width 0.3) (layer F.Cu) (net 18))
 (segment (start 85.65 109.25) (end 91.15 109.25) (width 0.3) (layer F.Cu) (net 18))
 (segment (start 84.65 110.25) (end 85.65 109.25) (width 0.3) (layer F.Cu) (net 18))
 (segment (start 80.85 110.75) (end 84.9 110.75) (width 0.3) (layer F.Cu) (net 17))
 (segment (start 91.15 109.748002) (end 91.15 109.75) (width 0.3) (layer F.Cu) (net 17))
 (segment (start 85.901998 109.748002) (end 91.15 109.748002) (width 0.3) (layer F.Cu) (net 17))
 (segment (start 84.9 110.75) (end 85.901998 109.748002) (width 0.3) (layer F.Cu) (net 17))
 (segment (start 80.85 111.25) (end 85.90042 111.25) (width 0.3) (layer F.Cu) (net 3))
 (segment (start 85.90042 111.25) (end 86.45042 110.7) (width 0.3) (layer F.Cu) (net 3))
 (segment (start 80.85 111.75) (end 86.95 111.75) (width 0.3) (layer F.Cu) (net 4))
 (segment (start 87.34958 111.35042) (end 87.34958 110.7) (width 0.3) (layer F.Cu) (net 4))
 (segment (start 86.95 111.75) (end 87.34958 111.35042) (width 0.3) (layer F.Cu) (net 4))
 (segment (start 91.15 111.25) (end 88.945718 111.25) (width 0.3) (layer F.Cu) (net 16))
 (segment (start 80.85 112.251998) (end 80.85 112.25) (width 0.3) (layer F.Cu) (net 16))
 (segment (start 87.94372 112.251998) (end 80.85 112.251998) (width 0.3) (layer F.Cu) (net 16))
 (segment (start 88.945718 111.25) (end 87.94372 112.251998) (width 0.3) (layer F.Cu) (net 16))
 (segment (start 80.85 112.75) (end 88.25 112.75) (width 0.3) (layer F.Cu) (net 15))
 (segment (start 91.15 111.751998) (end 91.15 111.75) (width 0.3) (layer F.Cu) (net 15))
 (segment (start 89.248002 111.751998) (end 91.15 111.751998) (width 0.3) (layer F.Cu) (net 15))
 (segment (start 88.25 112.75) (end 89.248002 111.751998) (width 0.3) (layer F.Cu) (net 15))
 (segment (start 91.15 112.25) (end 89.95 112.25) (width 0.3) (layer F.Cu) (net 13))
 (segment (start 80.85 115.251998) (end 80.85 115.25) (width 0.3) (layer F.Cu) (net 13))
 (segment (start 79.148002 115.251998) (end 80.85 115.251998) (width 0.3) (layer F.Cu) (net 13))
 (segment (start 79.1 115.3) (end 79.148002 115.251998) (width 0.3) (layer F.Cu) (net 13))
 (via (at 79.1 115.3) (size 0.889) (layers F.Cu B.Cu) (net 13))
 (segment (start 79.1 113.7) (end 79.1 115.3) (width 0.3) (layer B.Cu) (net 13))
 (segment (start 80.1 112.7) (end 79.1 113.7) (width 0.3) (layer B.Cu) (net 13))
 (segment (start 89.5 112.7) (end 80.1 112.7) (width 0.3) (layer B.Cu) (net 13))
 (via (at 89.5 112.7) (size 0.889) (layers F.Cu B.Cu) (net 13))
 (segment (start 89.95 112.25) (end 89.5 112.7) (width 0.3) (layer F.Cu) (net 13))
 (segment (start 80.85 115.75) (end 82.75 115.75) (width 0.3) (layer F.Cu) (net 12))
 (segment (start 92.85 112.75) (end 91.15 112.75) (width 0.3) (layer F.Cu) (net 12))
 (segment (start 92.9 112.8) (end 92.85 112.75) (width 0.3) (layer F.Cu) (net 12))
 (via (at 92.9 112.8) (size 0.889) (layers F.Cu B.Cu) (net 12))
 (segment (start 92.9 114) (end 92.9 112.8) (width 0.3) (layer B.Cu) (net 12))
 (segment (start 91.6 115.3) (end 92.9 114) (width 0.3) (layer B.Cu) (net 12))
 (segment (start 83.2 115.3) (end 91.6 115.3) (width 0.3) (layer B.Cu) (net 12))
 (via (at 83.2 115.3) (size 0.889) (layers F.Cu B.Cu) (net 12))
 (segment (start 82.75 115.75) (end 83.2 115.3) (width 0.3) (layer F.Cu) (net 12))
 (segment (start 80.85 116.25) (end 83.845718 116.25) (width 0.3) (layer F.Cu) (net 11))
 (segment (start 91.15 115.251998) (end 91.15 115.25) (width 0.3) (layer F.Cu) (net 11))
 (segment (start 84.84372 115.251998) (end 91.15 115.251998) (width 0.3) (layer F.Cu) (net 11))
 (segment (start 83.845718 116.25) (end 84.84372 115.251998) (width 0.3) (layer F.Cu) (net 11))
 (segment (start 80.85 116.75) (end 84.05 116.75) (width 0.3) (layer F.Cu) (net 9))
 (segment (start 85.05 115.75) (end 91.15 115.75) (width 0.3) (layer F.Cu) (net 9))
 (segment (start 84.05 116.75) (end 85.05 115.75) (width 0.3) (layer F.Cu) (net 9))
 (segment (start 96 111.75) (end 92.95 111.75) (width 0.3) (layer F.Cu) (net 7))
 (segment (start 92.95 111.75) (end 92.7 111.5) (width 0.3) (layer F.Cu) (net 7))
 (segment (start 96.85 111.25) (end 96.85 111.751998) (width 0.3) (layer F.Cu) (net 7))
 (segment (start 96.85 111.751998) (end 96.85 111.75) (width 0.3) (layer F.Cu) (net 7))
 (segment (start 91.15 110.25) (end 91.15 110.751998) (width 0.3) (layer F.Cu) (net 7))
 (segment (start 91.15 110.751998) (end 91.15 110.75) (width 0.3) (layer F.Cu) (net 7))
 (segment (start 75.15 109.25) (end 75.15 109.75) (width 0.3) (layer F.Cu) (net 7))
 (segment (start 75.15 117.25) (end 75.15 117.75) (width 0.3) (layer F.Cu) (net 7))
 (segment (start 75.15 117.75) (end 73.45 117.75) (width 0.3) (layer F.Cu) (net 7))
 (segment (start 73.45 117.75) (end 71.9 116.2) (width 0.3) (layer F.Cu) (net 7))
 (via (at 71.9 116.2) (size 0.889) (layers F.Cu B.Cu) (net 7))
 (segment (start 71.9 116.2) (end 73.2 116.2) (width 0.3) (layer B.Cu) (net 7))
 (segment (start 73.2 116.2) (end 77.9 111.5) (width 0.3) (layer B.Cu) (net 7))
 (segment (start 77.9 111.5) (end 92.7 111.5) (width 0.3) (layer B.Cu) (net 7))
 (via (at 92.7 111.5) (size 0.889) (layers F.Cu B.Cu) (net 7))
 (segment (start 91.951998 110.751998) (end 91.15 110.751998) (width 0.3) (layer F.Cu) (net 7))
 (segment (start 92.7 111.5) (end 91.951998 110.751998) (width 0.3) (layer F.Cu) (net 7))
 (segment (start 91.15 110.751998) (end 91.15 110.75) (width 0.3) (layer F.Cu) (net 7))
 (segment (start 75.15 117.25) (end 73.85 117.25) (width 0.3) (layer F.Cu) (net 7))
 (segment (start 88.75 110.25) (end 91.15 110.25) (width 0.3) (layer F.Cu) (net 7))
 (segment (start 88.4 110.6) (end 88.75 110.25) (width 0.3) (layer F.Cu) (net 7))
 (via (at 88.4 110.6) (size 0.889) (layers F.Cu B.Cu) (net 7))
 (segment (start 77 110.6) (end 88.4 110.6) (width 0.3) (layer B.Cu) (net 7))
 (segment (start 73.2 114.4) (end 77 110.6) (width 0.3) (layer B.Cu) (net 7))
 (via (at 73.2 114.4) (size 0.889) (layers F.Cu B.Cu) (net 7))
 (segment (start 73.2 116.6) (end 73.2 114.4) (width 0.3) (layer F.Cu) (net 7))
 (segment (start 73.85 117.25) (end 73.2 116.6) (width 0.3) (layer F.Cu) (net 7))
 (segment (start 75.15 109.25) (end 78.35 109.25) (width 0.3) (layer F.Cu) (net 7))
 (segment (start 95.45 111.25) (end 96.85 111.25) (width 0.3) (layer F.Cu) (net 7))
 (segment (start 91.3 107.1) (end 95.45 111.25) (width 0.3) (layer F.Cu) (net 7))
 (segment (start 80.5 107.1) (end 91.3 107.1) (width 0.3) (layer F.Cu) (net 7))
 (segment (start 78.35 109.25) (end 80.5 107.1) (width 0.3) (layer F.Cu) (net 7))
 (segment (start 75.15 109.75) (end 78.55 109.75) (width 0.3) (layer F.Cu) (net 7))
 (segment (start 91 107.6) (end 95.15 111.75) (width 0.3) (layer F.Cu) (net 7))
 (segment (start 80.7 107.6) (end 91 107.6) (width 0.3) (layer F.Cu) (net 7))
 (segment (start 78.55 109.75) (end 80.7 107.6) (width 0.3) (layer F.Cu) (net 7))
 (segment (start 95.15 111.75) (end 96 111.75) (width 0.3) (layer F.Cu) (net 7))
 (segment (start 96 111.75) (end 96.85 111.75) (width 0.3) (layer F.Cu) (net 7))
 (segment (start 96.85 116.25) (end 96.85 116.75) (width 0.3) (layer F.Cu) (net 10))
 (segment (start 91.15 117.25) (end 91.15 117.751998) (width 0.3) (layer F.Cu) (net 10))
 (segment (start 91.15 117.751998) (end 91.15 117.75) (width 0.3) (layer F.Cu) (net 10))
 (segment (start 75.15 115.25) (end 75.15 115.75) (width 0.3) (layer F.Cu) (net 10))
 (segment (start 75.15 115.75) (end 75.15 116.25) (width 0.3) (layer F.Cu) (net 10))
 (segment (start 75.15 116.75) (end 75.15 116.25) (width 0.3) (layer F.Cu) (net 10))
 (segment (start 75.15 116.75) (end 76.15 116.75) (width 0.3) (layer F.Cu) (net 10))
 (segment (start 76.15 116.75) (end 81.1 121.7) (width 0.3) (layer F.Cu) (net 10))
 (segment (start 81.1 121.7) (end 84.7 121.7) (width 0.3) (layer F.Cu) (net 10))
 (segment (start 84.7 121.7) (end 88.648002 117.751998) (width 0.3) (layer F.Cu) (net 10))
 (segment (start 88.648002 117.751998) (end 91.15 117.751998) (width 0.3) (layer F.Cu) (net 10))
 (segment (start 91.15 117.751998) (end 91.15 117.75) (width 0.3) (layer F.Cu) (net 10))
 (segment (start 75.15 116.25) (end 76.35 116.25) (width 0.3) (layer F.Cu) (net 10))
 (segment (start 88.45 117.25) (end 91.15 117.25) (width 0.3) (layer F.Cu) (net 10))
 (segment (start 84.6 121.1) (end 88.45 117.25) (width 0.3) (layer F.Cu) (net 10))
 (segment (start 81.2 121.1) (end 84.6 121.1) (width 0.3) (layer F.Cu) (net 10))
 (segment (start 76.35 116.25) (end 81.2 121.1) (width 0.3) (layer F.Cu) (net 10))
 (segment (start 75.15 115.75) (end 76.35 115.75) (width 0.3) (layer F.Cu) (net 10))
 (segment (start 93.55 116.75) (end 96.85 116.75) (width 0.3) (layer F.Cu) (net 10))
 (segment (start 93.2 117.1) (end 93.55 116.75) (width 0.3) (layer F.Cu) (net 10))
 (via (at 93.2 117.1) (size 0.889) (layers F.Cu B.Cu) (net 10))
 (segment (start 78.3 117.1) (end 93.2 117.1) (width 0.3) (layer B.Cu) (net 10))
 (segment (start 78.2 117) (end 78.3 117.1) (width 0.3) (layer B.Cu) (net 10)) (via (at 78.2 117) (size 0.889) (layers F.Cu B.Cu) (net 10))
 (segment (start 76.35 115.75) (end 78.2 117) (width 0.3) (layer F.Cu) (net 10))
 (segment (start 75.15 115.25) (end 77.25 115.25) (width 0.3) (layer F.Cu) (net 10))
 (segment (start 94.05 116.25) (end 96.85 116.25) (width 0.3) (layer F.Cu) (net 10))
 (segment (start 93.2 115.4) (end 94.05 116.25) (width 0.3) (layer F.Cu) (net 10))
 (via (at 93.2 115.4) (size 0.889) (layers F.Cu B.Cu) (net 10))
 (segment (start 92.3 116.3) (end 93.2 115.4) (width 0.3) (layer B.Cu) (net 10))
 (segment (start 78.3 116.3) (end 92.3 116.3) (width 0.3) (layer B.Cu) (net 10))
 (segment (start 77.7 115.3) (end 78.3 116.3) (width 0.3) (layer B.Cu) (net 10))
 (via (at 77.7 115.3) (size 0.889) (layers F.Cu B.Cu) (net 10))
 (segment (start 77.25 115.25) (end 77.7 115.3) (width 0.3) (layer F.Cu) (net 10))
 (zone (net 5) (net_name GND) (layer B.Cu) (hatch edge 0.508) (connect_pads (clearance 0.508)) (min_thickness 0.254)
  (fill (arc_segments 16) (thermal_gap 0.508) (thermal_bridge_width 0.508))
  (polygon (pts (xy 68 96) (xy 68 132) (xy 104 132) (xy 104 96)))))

